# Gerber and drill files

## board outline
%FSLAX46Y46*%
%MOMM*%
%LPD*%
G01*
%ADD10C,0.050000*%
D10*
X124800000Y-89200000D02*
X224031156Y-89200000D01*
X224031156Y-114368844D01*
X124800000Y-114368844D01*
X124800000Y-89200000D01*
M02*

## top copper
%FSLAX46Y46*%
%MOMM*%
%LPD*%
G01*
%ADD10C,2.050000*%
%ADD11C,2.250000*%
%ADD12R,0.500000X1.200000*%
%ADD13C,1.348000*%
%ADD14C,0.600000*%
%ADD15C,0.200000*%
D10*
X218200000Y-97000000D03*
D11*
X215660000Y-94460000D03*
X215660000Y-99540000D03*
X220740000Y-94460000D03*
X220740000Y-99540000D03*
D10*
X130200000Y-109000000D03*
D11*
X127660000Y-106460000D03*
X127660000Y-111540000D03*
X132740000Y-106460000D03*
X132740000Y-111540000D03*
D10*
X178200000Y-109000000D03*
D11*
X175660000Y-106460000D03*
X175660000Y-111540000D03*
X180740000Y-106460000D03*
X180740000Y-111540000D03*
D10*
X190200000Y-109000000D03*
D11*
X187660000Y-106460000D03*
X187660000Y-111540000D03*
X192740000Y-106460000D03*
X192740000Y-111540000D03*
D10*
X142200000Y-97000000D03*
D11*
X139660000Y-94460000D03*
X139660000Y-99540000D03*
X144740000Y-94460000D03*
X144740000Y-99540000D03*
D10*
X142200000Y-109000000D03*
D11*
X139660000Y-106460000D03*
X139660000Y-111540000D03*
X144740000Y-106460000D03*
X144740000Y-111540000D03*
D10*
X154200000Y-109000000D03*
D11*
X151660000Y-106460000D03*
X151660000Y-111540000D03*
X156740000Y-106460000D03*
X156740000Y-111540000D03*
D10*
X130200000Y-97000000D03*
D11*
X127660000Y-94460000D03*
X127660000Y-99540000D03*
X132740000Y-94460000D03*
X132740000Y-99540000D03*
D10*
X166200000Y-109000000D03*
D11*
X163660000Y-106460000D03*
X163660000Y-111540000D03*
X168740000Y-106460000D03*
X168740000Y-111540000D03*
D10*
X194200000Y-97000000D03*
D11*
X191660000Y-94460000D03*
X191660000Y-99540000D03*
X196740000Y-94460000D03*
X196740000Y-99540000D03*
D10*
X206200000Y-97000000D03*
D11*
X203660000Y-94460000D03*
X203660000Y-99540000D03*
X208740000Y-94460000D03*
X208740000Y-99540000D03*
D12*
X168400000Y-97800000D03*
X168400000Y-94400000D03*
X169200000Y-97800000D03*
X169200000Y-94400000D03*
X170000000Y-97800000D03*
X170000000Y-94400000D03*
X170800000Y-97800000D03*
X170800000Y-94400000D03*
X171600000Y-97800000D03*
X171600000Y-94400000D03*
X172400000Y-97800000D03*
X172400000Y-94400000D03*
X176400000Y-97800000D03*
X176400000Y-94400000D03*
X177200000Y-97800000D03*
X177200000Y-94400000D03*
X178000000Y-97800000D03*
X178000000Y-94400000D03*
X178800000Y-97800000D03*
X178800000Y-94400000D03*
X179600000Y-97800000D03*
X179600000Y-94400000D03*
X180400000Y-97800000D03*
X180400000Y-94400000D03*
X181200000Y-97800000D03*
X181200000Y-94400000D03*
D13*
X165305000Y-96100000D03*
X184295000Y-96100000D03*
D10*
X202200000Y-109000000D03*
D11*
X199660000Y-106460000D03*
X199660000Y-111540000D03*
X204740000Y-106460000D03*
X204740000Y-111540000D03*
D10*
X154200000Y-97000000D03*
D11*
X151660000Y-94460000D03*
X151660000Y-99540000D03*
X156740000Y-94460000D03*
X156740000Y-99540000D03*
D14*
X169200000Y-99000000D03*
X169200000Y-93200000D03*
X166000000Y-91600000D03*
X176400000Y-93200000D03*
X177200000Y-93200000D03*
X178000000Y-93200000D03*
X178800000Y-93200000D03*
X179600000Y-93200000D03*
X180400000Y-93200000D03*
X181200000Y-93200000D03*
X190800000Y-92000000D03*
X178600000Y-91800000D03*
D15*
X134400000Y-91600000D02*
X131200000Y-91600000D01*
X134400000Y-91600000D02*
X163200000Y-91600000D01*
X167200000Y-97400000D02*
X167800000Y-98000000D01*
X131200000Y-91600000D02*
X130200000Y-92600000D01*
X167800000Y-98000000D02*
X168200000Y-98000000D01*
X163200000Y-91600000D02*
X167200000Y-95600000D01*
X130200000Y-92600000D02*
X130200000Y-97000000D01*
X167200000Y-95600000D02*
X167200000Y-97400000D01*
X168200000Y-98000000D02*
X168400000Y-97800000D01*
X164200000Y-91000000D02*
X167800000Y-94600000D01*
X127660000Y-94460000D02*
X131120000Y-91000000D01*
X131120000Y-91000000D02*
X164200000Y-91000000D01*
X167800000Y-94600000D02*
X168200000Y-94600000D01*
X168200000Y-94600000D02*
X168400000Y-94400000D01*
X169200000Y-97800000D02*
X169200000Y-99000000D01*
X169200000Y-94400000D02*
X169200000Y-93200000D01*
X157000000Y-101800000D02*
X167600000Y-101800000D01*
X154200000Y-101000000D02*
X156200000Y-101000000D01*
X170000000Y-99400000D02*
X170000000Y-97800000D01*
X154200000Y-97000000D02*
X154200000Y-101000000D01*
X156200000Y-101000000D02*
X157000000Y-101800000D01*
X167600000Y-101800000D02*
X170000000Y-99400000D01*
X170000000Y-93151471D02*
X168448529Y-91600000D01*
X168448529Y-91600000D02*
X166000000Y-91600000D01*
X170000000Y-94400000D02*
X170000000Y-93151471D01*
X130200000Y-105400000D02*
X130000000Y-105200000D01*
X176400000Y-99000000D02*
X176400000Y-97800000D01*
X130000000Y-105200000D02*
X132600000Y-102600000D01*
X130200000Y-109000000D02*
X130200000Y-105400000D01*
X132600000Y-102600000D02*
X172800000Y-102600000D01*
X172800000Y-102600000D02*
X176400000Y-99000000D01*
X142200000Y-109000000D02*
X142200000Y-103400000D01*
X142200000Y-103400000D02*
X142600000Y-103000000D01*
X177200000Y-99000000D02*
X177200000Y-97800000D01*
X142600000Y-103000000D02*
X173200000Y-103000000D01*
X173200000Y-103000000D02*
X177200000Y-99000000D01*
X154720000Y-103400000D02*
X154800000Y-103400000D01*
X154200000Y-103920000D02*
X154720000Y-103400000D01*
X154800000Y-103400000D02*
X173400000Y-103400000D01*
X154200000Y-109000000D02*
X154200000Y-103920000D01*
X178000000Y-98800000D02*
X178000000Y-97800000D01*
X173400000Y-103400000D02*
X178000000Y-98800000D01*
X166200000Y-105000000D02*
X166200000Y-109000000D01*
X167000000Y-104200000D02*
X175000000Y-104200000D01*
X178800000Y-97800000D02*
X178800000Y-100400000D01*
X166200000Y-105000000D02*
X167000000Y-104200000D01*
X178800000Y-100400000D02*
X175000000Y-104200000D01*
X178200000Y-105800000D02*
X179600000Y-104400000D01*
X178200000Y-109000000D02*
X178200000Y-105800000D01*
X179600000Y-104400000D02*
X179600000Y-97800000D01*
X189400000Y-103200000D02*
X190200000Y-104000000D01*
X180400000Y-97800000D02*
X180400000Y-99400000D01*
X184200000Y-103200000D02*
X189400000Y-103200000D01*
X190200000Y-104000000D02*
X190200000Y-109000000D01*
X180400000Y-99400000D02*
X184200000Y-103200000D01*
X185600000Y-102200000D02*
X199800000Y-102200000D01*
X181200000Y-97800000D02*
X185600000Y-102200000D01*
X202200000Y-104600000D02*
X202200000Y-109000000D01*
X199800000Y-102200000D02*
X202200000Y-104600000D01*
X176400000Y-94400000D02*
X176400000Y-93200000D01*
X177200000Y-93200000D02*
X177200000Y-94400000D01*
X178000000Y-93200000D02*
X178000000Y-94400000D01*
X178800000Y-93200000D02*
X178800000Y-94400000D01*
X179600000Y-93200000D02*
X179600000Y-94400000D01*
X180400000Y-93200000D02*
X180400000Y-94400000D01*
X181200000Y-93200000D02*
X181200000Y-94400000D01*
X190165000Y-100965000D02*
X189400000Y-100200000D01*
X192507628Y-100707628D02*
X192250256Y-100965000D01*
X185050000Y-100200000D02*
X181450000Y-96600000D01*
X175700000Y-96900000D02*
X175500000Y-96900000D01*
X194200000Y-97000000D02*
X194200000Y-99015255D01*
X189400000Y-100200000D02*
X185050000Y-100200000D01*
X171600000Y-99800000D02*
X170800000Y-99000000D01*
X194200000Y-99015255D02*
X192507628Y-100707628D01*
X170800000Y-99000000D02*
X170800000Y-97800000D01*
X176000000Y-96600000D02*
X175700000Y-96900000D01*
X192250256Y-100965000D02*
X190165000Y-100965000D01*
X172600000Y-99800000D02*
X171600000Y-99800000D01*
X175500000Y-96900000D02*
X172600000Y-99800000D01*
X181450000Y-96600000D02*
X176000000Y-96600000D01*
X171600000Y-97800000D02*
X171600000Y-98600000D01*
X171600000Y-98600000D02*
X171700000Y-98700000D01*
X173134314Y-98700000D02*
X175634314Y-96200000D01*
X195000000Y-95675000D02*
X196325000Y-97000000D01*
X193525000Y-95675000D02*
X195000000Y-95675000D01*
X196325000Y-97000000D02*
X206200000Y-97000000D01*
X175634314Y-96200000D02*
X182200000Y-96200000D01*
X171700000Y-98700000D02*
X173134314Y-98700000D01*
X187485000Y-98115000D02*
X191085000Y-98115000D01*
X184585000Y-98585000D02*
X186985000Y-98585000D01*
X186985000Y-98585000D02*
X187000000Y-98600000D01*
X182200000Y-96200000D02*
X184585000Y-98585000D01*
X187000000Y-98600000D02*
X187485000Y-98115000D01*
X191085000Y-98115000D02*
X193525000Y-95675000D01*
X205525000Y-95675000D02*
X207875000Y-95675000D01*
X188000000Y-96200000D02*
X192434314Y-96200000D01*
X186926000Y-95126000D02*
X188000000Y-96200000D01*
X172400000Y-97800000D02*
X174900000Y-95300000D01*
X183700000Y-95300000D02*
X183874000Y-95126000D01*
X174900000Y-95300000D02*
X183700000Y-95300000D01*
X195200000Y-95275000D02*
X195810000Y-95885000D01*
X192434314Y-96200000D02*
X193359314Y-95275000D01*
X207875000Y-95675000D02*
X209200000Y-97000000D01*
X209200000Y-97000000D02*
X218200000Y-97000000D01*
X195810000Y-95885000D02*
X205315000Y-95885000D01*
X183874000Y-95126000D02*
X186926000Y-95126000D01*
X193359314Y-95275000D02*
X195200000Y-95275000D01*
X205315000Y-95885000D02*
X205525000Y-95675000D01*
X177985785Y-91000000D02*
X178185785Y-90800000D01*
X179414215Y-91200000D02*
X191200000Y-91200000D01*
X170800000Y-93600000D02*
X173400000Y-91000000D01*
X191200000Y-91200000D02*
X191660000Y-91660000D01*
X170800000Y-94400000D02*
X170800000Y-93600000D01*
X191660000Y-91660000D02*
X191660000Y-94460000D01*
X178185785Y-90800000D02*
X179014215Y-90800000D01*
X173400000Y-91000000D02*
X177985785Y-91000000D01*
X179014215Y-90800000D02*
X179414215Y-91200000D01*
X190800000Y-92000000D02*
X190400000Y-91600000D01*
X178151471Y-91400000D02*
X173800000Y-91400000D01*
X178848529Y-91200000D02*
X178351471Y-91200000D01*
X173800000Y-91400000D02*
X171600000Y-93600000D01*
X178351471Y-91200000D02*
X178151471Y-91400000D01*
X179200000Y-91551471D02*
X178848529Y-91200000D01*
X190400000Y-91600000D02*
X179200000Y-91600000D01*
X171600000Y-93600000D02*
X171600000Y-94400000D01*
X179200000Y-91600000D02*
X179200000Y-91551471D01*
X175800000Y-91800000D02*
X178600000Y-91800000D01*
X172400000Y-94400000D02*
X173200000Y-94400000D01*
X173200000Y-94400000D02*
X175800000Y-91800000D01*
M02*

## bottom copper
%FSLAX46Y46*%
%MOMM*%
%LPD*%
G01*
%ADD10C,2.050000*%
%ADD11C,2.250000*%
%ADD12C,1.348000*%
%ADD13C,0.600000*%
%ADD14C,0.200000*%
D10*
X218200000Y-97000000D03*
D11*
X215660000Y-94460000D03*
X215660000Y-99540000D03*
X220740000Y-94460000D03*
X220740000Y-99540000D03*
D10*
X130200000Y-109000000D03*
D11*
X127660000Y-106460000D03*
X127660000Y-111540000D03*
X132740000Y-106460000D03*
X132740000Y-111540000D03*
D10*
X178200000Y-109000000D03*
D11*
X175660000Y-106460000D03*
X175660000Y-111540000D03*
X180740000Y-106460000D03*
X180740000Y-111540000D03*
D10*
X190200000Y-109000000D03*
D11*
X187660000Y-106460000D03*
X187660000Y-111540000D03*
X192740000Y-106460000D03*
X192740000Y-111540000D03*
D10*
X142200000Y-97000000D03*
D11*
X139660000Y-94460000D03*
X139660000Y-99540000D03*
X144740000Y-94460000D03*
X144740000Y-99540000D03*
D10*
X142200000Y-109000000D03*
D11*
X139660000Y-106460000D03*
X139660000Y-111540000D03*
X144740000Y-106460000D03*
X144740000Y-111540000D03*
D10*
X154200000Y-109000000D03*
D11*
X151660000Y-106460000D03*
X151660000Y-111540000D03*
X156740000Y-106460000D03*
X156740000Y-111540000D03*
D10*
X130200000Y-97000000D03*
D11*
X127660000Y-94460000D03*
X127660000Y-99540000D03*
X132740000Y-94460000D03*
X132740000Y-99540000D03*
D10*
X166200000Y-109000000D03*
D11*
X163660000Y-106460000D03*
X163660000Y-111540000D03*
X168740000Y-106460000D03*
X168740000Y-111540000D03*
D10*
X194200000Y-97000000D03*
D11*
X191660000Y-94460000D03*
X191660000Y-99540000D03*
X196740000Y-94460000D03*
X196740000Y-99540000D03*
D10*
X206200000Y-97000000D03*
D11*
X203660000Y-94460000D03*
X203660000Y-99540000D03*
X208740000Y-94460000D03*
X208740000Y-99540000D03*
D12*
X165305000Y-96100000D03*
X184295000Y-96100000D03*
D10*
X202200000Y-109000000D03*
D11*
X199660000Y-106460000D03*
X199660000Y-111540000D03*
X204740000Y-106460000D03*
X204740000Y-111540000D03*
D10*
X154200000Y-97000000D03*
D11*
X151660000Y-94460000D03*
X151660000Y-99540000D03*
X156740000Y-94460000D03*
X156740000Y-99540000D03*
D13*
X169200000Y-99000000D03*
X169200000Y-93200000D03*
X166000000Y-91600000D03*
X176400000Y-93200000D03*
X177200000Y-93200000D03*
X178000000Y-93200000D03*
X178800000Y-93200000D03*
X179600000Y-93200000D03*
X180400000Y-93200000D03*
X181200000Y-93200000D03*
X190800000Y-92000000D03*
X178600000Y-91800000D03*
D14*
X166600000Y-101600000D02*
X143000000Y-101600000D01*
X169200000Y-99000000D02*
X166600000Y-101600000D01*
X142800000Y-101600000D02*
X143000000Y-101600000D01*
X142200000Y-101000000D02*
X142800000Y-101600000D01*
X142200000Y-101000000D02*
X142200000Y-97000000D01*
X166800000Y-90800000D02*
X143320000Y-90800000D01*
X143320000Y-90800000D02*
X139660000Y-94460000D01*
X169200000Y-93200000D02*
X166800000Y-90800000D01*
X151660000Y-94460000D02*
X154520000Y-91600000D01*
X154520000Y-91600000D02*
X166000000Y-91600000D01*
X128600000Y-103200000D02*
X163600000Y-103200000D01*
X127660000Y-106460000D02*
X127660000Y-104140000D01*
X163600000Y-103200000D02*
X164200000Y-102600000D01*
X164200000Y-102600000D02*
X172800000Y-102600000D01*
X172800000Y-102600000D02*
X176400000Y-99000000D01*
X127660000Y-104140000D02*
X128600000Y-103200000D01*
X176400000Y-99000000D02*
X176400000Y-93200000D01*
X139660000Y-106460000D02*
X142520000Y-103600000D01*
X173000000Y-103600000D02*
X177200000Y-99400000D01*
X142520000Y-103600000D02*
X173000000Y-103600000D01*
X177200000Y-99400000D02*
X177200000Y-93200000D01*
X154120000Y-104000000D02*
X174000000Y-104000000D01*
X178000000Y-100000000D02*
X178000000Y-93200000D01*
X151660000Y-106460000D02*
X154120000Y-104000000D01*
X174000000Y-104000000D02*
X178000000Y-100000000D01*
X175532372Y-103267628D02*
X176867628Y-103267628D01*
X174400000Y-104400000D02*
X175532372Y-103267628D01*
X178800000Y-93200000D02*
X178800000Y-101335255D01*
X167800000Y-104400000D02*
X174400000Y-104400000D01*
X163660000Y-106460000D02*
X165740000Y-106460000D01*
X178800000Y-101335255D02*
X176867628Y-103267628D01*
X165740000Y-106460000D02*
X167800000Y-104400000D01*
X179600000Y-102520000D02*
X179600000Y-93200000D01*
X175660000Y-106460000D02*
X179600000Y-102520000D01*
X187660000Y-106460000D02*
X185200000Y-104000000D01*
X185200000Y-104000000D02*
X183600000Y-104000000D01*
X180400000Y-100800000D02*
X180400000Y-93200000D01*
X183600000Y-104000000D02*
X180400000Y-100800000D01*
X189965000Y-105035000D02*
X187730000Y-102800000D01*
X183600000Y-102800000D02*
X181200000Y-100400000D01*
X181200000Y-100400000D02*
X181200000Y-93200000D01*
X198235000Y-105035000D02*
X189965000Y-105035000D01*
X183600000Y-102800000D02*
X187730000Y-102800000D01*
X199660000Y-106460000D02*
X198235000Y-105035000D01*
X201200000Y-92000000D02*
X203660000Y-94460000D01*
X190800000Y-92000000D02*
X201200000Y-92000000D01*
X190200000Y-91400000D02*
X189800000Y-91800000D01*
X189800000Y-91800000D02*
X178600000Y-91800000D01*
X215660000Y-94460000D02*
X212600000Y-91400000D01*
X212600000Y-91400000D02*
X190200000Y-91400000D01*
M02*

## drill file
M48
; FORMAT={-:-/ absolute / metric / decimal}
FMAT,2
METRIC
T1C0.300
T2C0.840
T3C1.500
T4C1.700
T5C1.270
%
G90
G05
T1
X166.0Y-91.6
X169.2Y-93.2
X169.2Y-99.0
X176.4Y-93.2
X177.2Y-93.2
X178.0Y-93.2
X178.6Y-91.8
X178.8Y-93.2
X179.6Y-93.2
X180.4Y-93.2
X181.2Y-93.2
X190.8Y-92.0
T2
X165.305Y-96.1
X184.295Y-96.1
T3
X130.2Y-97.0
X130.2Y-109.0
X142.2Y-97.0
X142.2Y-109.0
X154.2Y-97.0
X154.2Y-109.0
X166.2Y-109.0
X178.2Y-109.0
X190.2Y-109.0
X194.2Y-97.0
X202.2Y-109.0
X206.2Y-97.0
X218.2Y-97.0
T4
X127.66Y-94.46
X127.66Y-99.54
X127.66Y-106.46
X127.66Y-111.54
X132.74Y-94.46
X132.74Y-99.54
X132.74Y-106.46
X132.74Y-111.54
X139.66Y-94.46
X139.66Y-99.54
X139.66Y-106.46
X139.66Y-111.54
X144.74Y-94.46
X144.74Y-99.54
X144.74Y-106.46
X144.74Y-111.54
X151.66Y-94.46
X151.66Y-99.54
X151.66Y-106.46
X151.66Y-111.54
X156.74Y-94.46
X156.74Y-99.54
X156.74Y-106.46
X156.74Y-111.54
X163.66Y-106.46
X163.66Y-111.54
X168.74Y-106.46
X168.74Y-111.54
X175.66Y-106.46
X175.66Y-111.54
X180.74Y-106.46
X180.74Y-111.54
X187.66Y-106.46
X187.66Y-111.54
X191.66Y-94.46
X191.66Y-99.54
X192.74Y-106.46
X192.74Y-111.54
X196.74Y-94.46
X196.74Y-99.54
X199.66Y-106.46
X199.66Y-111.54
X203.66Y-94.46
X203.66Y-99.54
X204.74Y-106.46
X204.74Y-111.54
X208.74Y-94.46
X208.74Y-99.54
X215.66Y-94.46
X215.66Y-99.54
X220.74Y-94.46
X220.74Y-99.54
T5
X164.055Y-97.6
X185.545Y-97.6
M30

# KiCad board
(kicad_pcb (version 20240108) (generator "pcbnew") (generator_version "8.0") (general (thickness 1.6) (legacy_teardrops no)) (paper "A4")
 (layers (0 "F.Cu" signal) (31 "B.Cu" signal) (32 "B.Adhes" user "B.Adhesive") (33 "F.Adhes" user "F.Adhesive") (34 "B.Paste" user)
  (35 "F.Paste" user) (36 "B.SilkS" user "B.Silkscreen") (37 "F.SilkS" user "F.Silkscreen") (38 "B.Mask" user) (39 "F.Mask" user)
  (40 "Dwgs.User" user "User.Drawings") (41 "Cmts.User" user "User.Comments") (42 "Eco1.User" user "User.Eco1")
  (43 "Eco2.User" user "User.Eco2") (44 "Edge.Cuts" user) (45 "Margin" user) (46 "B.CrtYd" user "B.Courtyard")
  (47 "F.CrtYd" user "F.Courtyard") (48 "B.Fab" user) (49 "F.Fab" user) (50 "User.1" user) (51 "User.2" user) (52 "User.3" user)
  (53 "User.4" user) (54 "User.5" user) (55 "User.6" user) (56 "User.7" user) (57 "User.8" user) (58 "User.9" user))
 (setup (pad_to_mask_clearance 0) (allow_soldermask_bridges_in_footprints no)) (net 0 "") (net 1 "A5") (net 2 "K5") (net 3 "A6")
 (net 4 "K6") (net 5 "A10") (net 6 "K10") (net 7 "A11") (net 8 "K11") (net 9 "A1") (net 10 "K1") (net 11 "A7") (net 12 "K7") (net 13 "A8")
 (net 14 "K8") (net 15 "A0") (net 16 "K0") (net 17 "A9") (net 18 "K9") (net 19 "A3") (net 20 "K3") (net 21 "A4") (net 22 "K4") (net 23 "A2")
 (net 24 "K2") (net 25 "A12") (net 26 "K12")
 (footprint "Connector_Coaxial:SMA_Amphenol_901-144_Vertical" (layer "F.Cu") (at 218.2 97)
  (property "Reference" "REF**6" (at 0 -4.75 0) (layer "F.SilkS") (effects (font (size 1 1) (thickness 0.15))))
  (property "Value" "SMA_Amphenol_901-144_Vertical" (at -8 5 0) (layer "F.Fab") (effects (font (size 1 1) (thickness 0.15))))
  (pad "1" thru_hole circle (at 0 0) (size 2.05 2.05) (drill 1.5) (layers "*.Cu" "*.Mask") (remove_unused_layers no) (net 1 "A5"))
  (pad "2" thru_hole circle (at -2.54 -2.54) (size 2.25 2.25) (drill 1.7) (layers "*.Cu" "*.Mask") (remove_unused_layers no) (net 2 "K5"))
  (pad "2" thru_hole circle (at -2.54 2.54) (size 2.25 2.25) (drill 1.7) (layers "*.Cu" "*.Mask") (remove_unused_layers no))
  (pad "2" thru_hole circle (at 2.54 -2.54) (size 2.25 2.25) (drill 1.7) (layers "*.Cu" "*.Mask") (remove_unused_layers no))
  (pad "2" thru_hole circle (at 2.54 2.54) (size 2.25 2.25) (drill 1.7) (layers "*.Cu" "*.Mask") (remove_unused_layers no)))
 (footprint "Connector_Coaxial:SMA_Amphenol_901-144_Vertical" (layer "F.Cu") (at 130.2 109)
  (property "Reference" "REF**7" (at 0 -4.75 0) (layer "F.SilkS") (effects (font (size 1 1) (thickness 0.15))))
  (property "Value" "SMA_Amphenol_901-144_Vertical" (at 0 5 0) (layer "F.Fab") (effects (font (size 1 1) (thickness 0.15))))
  (pad "1" thru_hole circle (at 0 0) (size 2.05 2.05) (drill 1.5) (layers "*.Cu" "*.Mask") (remove_unused_layers no) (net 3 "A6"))
  (pad "2" thru_hole circle (at -2.54 -2.54) (size 2.25 2.25) (drill 1.7) (layers "*.Cu" "*.Mask") (remove_unused_layers no) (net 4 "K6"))
  (pad "2" thru_hole circle (at -2.54 2.54) (size 2.25 2.25) (drill 1.7) (layers "*.Cu" "*.Mask") (remove_unused_layers no))
  (pad "2" thru_hole circle (at 2.54 -2.54) (size 2.25 2.25) (drill 1.7) (layers "*.Cu" "*.Mask") (remove_unused_layers no))
  (pad "2" thru_hole circle (at 2.54 2.54) (size 2.25 2.25) (drill 1.7) (layers "*.Cu" "*.Mask") (remove_unused_layers no)))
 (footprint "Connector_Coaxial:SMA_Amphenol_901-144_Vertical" (layer "F.Cu") (at 178.2 109)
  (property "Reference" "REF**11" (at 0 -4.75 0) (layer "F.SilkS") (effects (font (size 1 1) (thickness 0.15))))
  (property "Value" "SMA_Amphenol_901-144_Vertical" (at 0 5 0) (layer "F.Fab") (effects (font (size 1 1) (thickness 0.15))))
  (pad "1" thru_hole circle (at 0 0) (size 2.05 2.05) (drill 1.5) (layers "*.Cu" "*.Mask") (remove_unused_layers no) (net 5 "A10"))
  (pad "2" thru_hole circle (at -2.54 -2.54) (size 2.25 2.25) (drill 1.7) (layers "*.Cu" "*.Mask") (remove_unused_layers no) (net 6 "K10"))
  (pad "2" thru_hole circle (at -2.54 2.54) (size 2.25 2.25) (drill 1.7) (layers "*.Cu" "*.Mask") (remove_unused_layers no))
  (pad "2" thru_hole circle (at 2.54 -2.54) (size 2.25 2.25) (drill 1.7) (layers "*.Cu" "*.Mask") (remove_unused_layers no))
  (pad "2" thru_hole circle (at 2.54 2.54) (size 2.25 2.25) (drill 1.7) (layers "*.Cu" "*.Mask") (remove_unused_layers no)))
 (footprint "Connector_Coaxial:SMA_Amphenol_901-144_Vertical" (layer "F.Cu") (at 190.2 109)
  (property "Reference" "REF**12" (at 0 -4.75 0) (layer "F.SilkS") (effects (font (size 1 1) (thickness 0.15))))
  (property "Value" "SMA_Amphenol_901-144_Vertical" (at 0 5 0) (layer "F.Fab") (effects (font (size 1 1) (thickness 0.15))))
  (pad "1" thru_hole circle (at 0 0) (size 2.05 2.05) (drill 1.5) (layers "*.Cu" "*.Mask") (remove_unused_layers no) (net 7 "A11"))
  (pad "2" thru_hole circle (at -2.54 -2.54) (size 2.25 2.25) (drill 1.7) (layers "*.Cu" "*.Mask") (remove_unused_layers no) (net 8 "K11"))
  (pad "2" thru_hole circle (at -2.54 2.54) (size 2.25 2.25) (drill 1.7) (layers "*.Cu" "*.Mask") (remove_unused_layers no))
  (pad "2" thru_hole circle (at 2.54 -2.54) (size 2.25 2.25) (drill 1.7) (layers "*.Cu" "*.Mask") (remove_unused_layers no))
  (pad "2" thru_hole circle (at 2.54 2.54) (size 2.25 2.25) (drill 1.7) (layers "*.Cu" "*.Mask") (remove_unused_layers no)))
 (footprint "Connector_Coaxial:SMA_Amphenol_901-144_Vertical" (layer "F.Cu") (at 142.2 97)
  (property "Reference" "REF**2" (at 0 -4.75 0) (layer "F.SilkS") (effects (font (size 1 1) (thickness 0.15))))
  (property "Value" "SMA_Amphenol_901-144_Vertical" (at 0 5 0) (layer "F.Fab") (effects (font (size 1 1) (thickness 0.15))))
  (pad "1" thru_hole circle (at 0 0) (size 2.05 2.05) (drill 1.5) (layers "*.Cu" "*.Mask") (remove_unused_layers no) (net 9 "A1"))
  (pad "2" thru_hole circle (at -2.54 -2.54) (size 2.25 2.25) (drill 1.7) (layers "*.Cu" "*.Mask") (remove_unused_layers no) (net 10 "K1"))
  (pad "2" thru_hole circle (at -2.54 2.54) (size 2.25 2.25) (drill 1.7) (layers "*.Cu" "*.Mask") (remove_unused_layers no))
  (pad "2" thru_hole circle (at 2.54 -2.54) (size 2.25 2.25) (drill 1.7) (layers "*.Cu" "*.Mask") (remove_unused_layers no))
  (pad "2" thru_hole circle (at 2.54 2.54) (size 2.25 2.25) (drill 1.7) (layers "*.Cu" "*.Mask") (remove_unused_layers no)))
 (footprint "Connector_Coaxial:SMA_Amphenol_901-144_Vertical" (layer "F.Cu") (at 142.2 109)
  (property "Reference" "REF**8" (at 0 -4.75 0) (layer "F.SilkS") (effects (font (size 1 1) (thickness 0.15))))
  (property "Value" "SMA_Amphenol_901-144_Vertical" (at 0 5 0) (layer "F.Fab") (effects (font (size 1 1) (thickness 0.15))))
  (pad "1" thru_hole circle (at 0 0) (size 2.05 2.05) (drill 1.5) (layers "*.Cu" "*.Mask") (remove_unused_layers no) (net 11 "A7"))
  (pad "2" thru_hole circle (at -2.54 -2.54) (size 2.25 2.25) (drill 1.7) (layers "*.Cu" "*.Mask") (remove_unused_layers no) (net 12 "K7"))
  (pad "2" thru_hole circle (at -2.54 2.54) (size 2.25 2.25) (drill 1.7) (layers "*.Cu" "*.Mask") (remove_unused_layers no))
  (pad "2" thru_hole circle (at 2.54 -2.54) (size 2.25 2.25) (drill 1.7) (layers "*.Cu" "*.Mask") (remove_unused_layers no))
  (pad "2" thru_hole circle (at 2.54 2.54) (size 2.25 2.25) (drill 1.7) (layers "*.Cu" "*.Mask") (remove_unused_layers no)))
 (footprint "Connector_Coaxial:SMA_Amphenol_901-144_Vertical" (layer "F.Cu") (at 154.2 109)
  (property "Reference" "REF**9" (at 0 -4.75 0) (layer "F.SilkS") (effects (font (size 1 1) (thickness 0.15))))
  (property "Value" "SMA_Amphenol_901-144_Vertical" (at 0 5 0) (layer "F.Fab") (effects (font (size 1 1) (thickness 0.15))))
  (pad "1" thru_hole circle (at 0 0) (size 2.05 2.05) (drill 1.5) (layers "*.Cu" "*.Mask") (remove_unused_layers no) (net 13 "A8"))
  (pad "2" thru_hole circle (at -2.54 -2.54) (size 2.25 2.25) (drill 1.7) (layers "*.Cu" "*.Mask") (remove_unused_layers no) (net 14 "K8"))
  (pad "2" thru_hole circle (at -2.54 2.54) (size 2.25 2.25) (drill 1.7) (layers "*.Cu" "*.Mask") (remove_unused_layers no))
  (pad "2" thru_hole circle (at 2.54 -2.54) (size 2.25 2.25) (drill 1.7) (layers "*.Cu" "*.Mask") (remove_unused_layers no))
  (pad "2" thru_hole circle (at 2.54 2.54) (size 2.25 2.25) (drill 1.7) (layers "*.Cu" "*.Mask") (remove_unused_layers no)))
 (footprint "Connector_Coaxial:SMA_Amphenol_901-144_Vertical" (layer "F.Cu") (at 130.2 97)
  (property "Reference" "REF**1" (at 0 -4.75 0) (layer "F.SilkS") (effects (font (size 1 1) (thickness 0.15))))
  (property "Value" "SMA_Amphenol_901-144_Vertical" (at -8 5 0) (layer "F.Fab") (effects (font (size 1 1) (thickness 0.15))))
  (pad "1" thru_hole circle (at 0 0) (size 2.05 2.05) (drill 1.5) (layers "*.Cu" "*.Mask") (remove_unused_layers no) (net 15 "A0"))
  (pad "2" thru_hole circle (at -2.54 -2.54) (size 2.25 2.25) (drill 1.7) (layers "*.Cu" "*.Mask") (remove_unused_layers no) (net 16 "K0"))
  (pad "2" thru_hole circle (at -2.54 2.54) (size 2.25 2.25) (drill 1.7) (layers "*.Cu" "*.Mask") (remove_unused_layers no))
  (pad "2" thru_hole circle (at 2.54 -2.54) (size 2.25 2.25) (drill 1.7) (layers "*.Cu" "*.Mask") (remove_unused_layers no))
  (pad "2" thru_hole circle (at 2.54 2.54) (size 2.25 2.25) (drill 1.7) (layers "*.Cu" "*.Mask") (remove_unused_layers no)))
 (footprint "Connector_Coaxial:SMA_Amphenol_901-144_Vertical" (layer "F.Cu") (at 166.2 109)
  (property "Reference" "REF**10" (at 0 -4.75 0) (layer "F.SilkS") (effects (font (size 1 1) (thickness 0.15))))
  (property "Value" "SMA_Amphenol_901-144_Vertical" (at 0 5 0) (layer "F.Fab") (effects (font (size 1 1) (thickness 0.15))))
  (pad "1" thru_hole circle (at 0 0) (size 2.05 2.05) (drill 1.5) (layers "*.Cu" "*.Mask") (remove_unused_layers no) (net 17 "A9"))
  (pad "2" thru_hole circle (at -2.54 -2.54) (size 2.25 2.25) (drill 1.7) (layers "*.Cu" "*.Mask") (remove_unused_layers no) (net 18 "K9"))
  (pad "2" thru_hole circle (at -2.54 2.54) (size 2.25 2.25) (drill 1.7) (layers "*.Cu" "*.Mask") (remove_unused_layers no))
  (pad "2" thru_hole circle (at 2.54 -2.54) (size 2.25 2.25) (drill 1.7) (layers "*.Cu" "*.Mask") (remove_unused_layers no))
  (pad "2" thru_hole circle (at 2.54 2.54) (size 2.25 2.25) (drill 1.7) (layers "*.Cu" "*.Mask") (remove_unused_layers no)))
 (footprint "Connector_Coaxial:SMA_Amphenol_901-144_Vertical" (layer "F.Cu") (at 194.2 97)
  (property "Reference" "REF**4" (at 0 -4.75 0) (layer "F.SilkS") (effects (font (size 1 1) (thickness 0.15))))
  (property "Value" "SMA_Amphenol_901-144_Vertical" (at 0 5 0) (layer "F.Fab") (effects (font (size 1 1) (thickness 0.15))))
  (pad "1" thru_hole circle (at 0 0) (size 2.05 2.05) (drill 1.5) (layers "*.Cu" "*.Mask") (remove_unused_layers no) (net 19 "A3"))
  (pad "2" thru_hole circle (at -2.54 -2.54) (size 2.25 2.25) (drill 1.7) (layers "*.Cu" "*.Mask") (remove_unused_layers no) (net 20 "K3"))
  (pad "2" thru_hole circle (at -2.54 2.54) (size 2.25 2.25) (drill 1.7) (layers "*.Cu" "*.Mask") (remove_unused_layers no))
  (pad "2" thru_hole circle (at 2.54 -2.54) (size 2.25 2.25) (drill 1.7) (layers "*.Cu" "*.Mask") (remove_unused_layers no))
  (pad "2" thru_hole circle (at 2.54 2.54) (size 2.25 2.25) (drill 1.7) (layers "*.Cu" "*.Mask") (remove_unused_layers no)))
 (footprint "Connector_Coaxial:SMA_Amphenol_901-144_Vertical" (layer "F.Cu") (at 206.2 97)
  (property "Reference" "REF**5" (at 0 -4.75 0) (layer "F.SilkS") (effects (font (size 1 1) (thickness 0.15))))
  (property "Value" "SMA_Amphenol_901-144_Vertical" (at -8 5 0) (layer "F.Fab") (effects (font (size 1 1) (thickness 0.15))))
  (pad "1" thru_hole circle (at 0 0) (size 2.05 2.05) (drill 1.5) (layers "*.Cu" "*.Mask") (remove_unused_layers no) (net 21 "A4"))
  (pad "2" thru_hole circle (at -2.54 -2.54) (size 2.25 2.25) (drill 1.7) (layers "*.Cu" "*.Mask") (remove_unused_layers no) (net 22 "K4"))
  (pad "2" thru_hole circle (at -2.54 2.54) (size 2.25 2.25) (drill 1.7) (layers "*.Cu" "*.Mask") (remove_unused_layers no))
  (pad "2" thru_hole circle (at 2.54 -2.54) (size 2.25 2.25) (drill 1.7) (layers "*.Cu" "*.Mask") (remove_unused_layers no))
  (pad "2" thru_hole circle (at 2.54 2.54) (size 2.25 2.25) (drill 1.7) (layers "*.Cu" "*.Mask") (remove_unused_layers no)))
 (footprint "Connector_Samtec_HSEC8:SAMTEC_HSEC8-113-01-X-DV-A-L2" (layer "F.Cu") (at 174.8 96.1)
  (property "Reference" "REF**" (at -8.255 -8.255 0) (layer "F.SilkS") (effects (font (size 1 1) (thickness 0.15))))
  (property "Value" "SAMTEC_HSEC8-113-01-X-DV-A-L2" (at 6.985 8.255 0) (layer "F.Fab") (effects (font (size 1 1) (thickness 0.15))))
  (pad "" np_thru_hole circle (at -10.745 1.5) (size 1.27 1.27) (drill 1.27) (layers "F&B.Cu" "*.Mask"))
  (pad "" np_thru_hole circle (at 10.745 1.5) (size 1.27 1.27) (drill 1.27) (layers "F&B.Cu" "*.Mask"))
  (pad "01" smd rect (at -6.4 1.7) (size 0.5 1.2) (layers "F.Cu" "F.Paste" "F.Mask") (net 15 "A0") (solder_mask_margin 0.102))
  (pad "02" smd rect (at -6.4 -1.7) (size 0.5 1.2) (layers "F.Cu" "F.Paste" "F.Mask") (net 16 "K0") (solder_mask_margin 0.102))
  (pad "02" smd rect (at -5.6 1.7) (size 0.5 1.2) (layers "F.Cu" "F.Paste" "F.Mask") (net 9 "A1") (solder_mask_margin 0.102))
  (pad "04" smd rect (at -5.6 -1.7) (size 0.5 1.2) (layers "F.Cu" "F.Paste" "F.Mask") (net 10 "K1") (solder_mask_margin 0.102))
  (pad "05" smd rect (at -4.8 1.7) (size 0.5 1.2) (layers "F.Cu" "F.Paste" "F.Mask") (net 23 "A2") (solder_mask_margin 0.102))
  (pad "06" smd rect (at -4.8 -1.7) (size 0.5 1.2) (layers "F.Cu" "F.Paste" "F.Mask") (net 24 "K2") (solder_mask_margin 0.102))
  (pad "07" smd rect (at -4 1.7) (size 0.5 1.2) (layers "F.Cu" "F.Paste" "F.Mask") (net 19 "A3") (solder_mask_margin 0.102))
  (pad "08" smd rect (at -4 -1.7) (size 0.5 1.2) (layers "F.Cu" "F.Paste" "F.Mask") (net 20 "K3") (solder_mask_margin 0.102))
  (pad "09" smd rect (at -3.2 1.7) (size 0.5 1.2) (layers "F.Cu" "F.Paste" "F.Mask") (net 21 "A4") (solder_mask_margin 0.102))
  (pad "10" smd rect (at -3.2 -1.7) (size 0.5 1.2) (layers "F.Cu" "F.Paste" "F.Mask") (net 22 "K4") (solder_mask_margin 0.102))
  (pad "11" smd rect (at -2.4 1.7) (size 0.5 1.2) (layers "F.Cu" "F.Paste" "F.Mask") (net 1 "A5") (solder_mask_margin 0.102))
  (pad "12" smd rect (at -2.4 -1.7) (size 0.5 1.2) (layers "F.Cu" "F.Paste" "F.Mask") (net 2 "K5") (solder_mask_margin 0.102))
  (pad "13" smd rect (at 1.6 1.7) (size 0.5 1.2) (layers "F.Cu" "F.Paste" "F.Mask") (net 3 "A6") (solder_mask_margin 0.102))
  (pad "14" smd rect (at 1.6 -1.7) (size 0.5 1.2) (layers "F.Cu" "F.Paste" "F.Mask") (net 4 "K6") (solder_mask_margin 0.102))
  (pad "15" smd rect (at 2.4 1.7) (size 0.5 1.2) (layers "F.Cu" "F.Paste" "F.Mask") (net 11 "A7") (solder_mask_margin 0.102))
  (pad "16" smd rect (at 2.4 -1.7) (size 0.5 1.2) (layers "F.Cu" "F.Paste" "F.Mask") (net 12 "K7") (solder_mask_margin 0.102))
  (pad "17" smd rect (at 3.2 1.7) (size 0.5 1.2) (layers "F.Cu" "F.Paste" "F.Mask") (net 13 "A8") (solder_mask_margin 0.102))
  (pad "18" smd rect (at 3.2 -1.7) (size 0.5 1.2) (layers "F.Cu" "F.Paste" "F.Mask") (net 14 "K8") (solder_mask_margin 0.102))
  (pad "19" smd rect (at 4 1.7) (size 0.5 1.2) (layers "F.Cu" "F.Paste" "F.Mask") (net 17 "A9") (solder_mask_margin 0.102))
  (pad "20" smd rect (at 4 -1.7) (size 0.5 1.2) (layers "F.Cu" "F.Paste" "F.Mask") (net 18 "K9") (solder_mask_margin 0.102))
  (pad "21" smd rect (at 4.8 1.7) (size 0.5 1.2) (layers "F.Cu" "F.Paste" "F.Mask") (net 5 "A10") (solder_mask_margin 0.102))
  (pad "22" smd rect (at 4.8 -1.7) (size 0.5 1.2) (layers "F.Cu" "F.Paste" "F.Mask") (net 6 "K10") (solder_mask_margin 0.102))
  (pad "23" smd rect (at 5.6 1.7) (size 0.5 1.2) (layers "F.Cu" "F.Paste" "F.Mask") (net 7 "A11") (solder_mask_margin 0.102))
  (pad "24" smd rect (at 5.6 -1.7) (size 0.5 1.2) (layers "F.Cu" "F.Paste" "F.Mask") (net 8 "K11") (solder_mask_margin 0.102))
  (pad "25" smd rect (at 6.4 1.7) (size 0.5 1.2) (layers "F.Cu" "F.Paste" "F.Mask") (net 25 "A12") (solder_mask_margin 0.102))
  (pad "26" smd rect (at 6.4 -1.7) (size 0.5 1.2) (layers "F.Cu" "F.Paste" "F.Mask") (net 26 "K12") (solder_mask_margin 0.102))
  (pad "S1" thru_hole circle (at -9.495 0) (size 1.348 1.348) (drill 0.84) (layers "*.Cu" "*.Mask") (remove_unused_layers no)
   (solder_mask_margin 0.102))
  (pad "S2" thru_hole circle (at 9.495 0) (size 1.348 1.348) (drill 0.84) (layers "*.Cu" "*.Mask") (remove_unused_layers no)
   (solder_mask_margin 0.102)))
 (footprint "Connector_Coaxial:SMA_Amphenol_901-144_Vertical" (layer "F.Cu") (at 202.2 109)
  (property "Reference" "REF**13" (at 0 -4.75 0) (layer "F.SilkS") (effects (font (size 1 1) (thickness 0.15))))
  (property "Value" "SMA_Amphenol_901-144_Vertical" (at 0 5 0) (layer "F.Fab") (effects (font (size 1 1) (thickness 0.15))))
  (pad "1" thru_hole circle (at 0 0) (size 2.05 2.05) (drill 1.5) (layers "*.Cu" "*.Mask") (remove_unused_layers no) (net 25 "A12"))
  (pad "2" thru_hole circle (at -2.54 -2.54) (size 2.25 2.25) (drill 1.7) (layers "*.Cu" "*.Mask") (remove_unused_layers no) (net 26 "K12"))
  (pad "2" thru_hole circle (at -2.54 2.54) (size 2.25 2.25) (drill 1.7) (layers "*.Cu" "*.Mask") (remove_unused_layers no))
  (pad "2" thru_hole circle (at 2.54 -2.54) (size 2.25 2.25) (drill 1.7) (layers "*.Cu" "*.Mask") (remove_unused_layers no))
  (pad "2" thru_hole circle (at 2.54 2.54) (size 2.25 2.25) (drill 1.7) (layers "*.Cu" "*.Mask") (remove_unused_layers no)))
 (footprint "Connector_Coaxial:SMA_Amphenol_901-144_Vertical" (layer "F.Cu") (at 154.2 97)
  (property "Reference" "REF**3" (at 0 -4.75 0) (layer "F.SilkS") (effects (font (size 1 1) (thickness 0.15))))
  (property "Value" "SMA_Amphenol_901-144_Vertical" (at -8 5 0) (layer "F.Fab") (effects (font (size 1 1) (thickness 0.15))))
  (pad "1" thru_hole circle (at 0 0) (size 2.05 2.05) (drill 1.5) (layers "*.Cu" "*.Mask") (remove_unused_layers no) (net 23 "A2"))
  (pad "2" thru_hole circle (at -2.54 -2.54) (size 2.25 2.25) (drill 1.7) (layers "*.Cu" "*.Mask") (remove_unused_layers no) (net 24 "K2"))
  (pad "2" thru_hole circle (at -2.54 2.54) (size 2.25 2.25) (drill 1.7) (layers "*.Cu" "*.Mask") (remove_unused_layers no))
  (pad "2" thru_hole circle (at 2.54 -2.54) (size 2.25 2.25) (drill 1.7) (layers "*.Cu" "*.Mask") (remove_unused_layers no))
  (pad "2" thru_hole circle (at 2.54 2.54) (size 2.25 2.25) (drill 1.7) (layers "*.Cu" "*.Mask") (remove_unused_layers no)))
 (gr_rect (start 124.8 89.2) (end 224.031156 114.368844) (stroke (width 0.05) (type default)) (fill none) (layer "Edge.Cuts"))
 (segment (start 134.4 91.6) (end 131.2 91.6) (width 0.2) (layer "F.Cu") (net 15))
 (segment (start 134.4 91.6) (end 163.2 91.6) (width 0.2) (layer "F.Cu") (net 15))
 (segment (start 167.2 97.4) (end 167.8 98) (width 0.2) (layer "F.Cu") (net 15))
 (segment (start 131.2 91.6) (end 130.2 92.6) (width 0.2) (layer "F.Cu") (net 15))
 (segment (start 167.8 98) (end 168.2 98) (width 0.2) (layer "F.Cu") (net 15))
 (segment (start 163.2 91.6) (end 167.2 95.6) (width 0.2) (layer "F.Cu") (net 15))
 (segment (start 130.2 92.6) (end 130.2 97) (width 0.2) (layer "F.Cu") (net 15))
 (segment (start 167.2 95.6) (end 167.2 97.4) (width 0.2) (layer "F.Cu") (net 15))
 (segment (start 168.2 98) (end 168.4 97.8) (width 0.2) (layer "F.Cu") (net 15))
 (segment (start 164.2 91) (end 167.8 94.6) (width 0.2) (layer "F.Cu") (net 16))
 (segment (start 127.66 94.46) (end 131.12 91) (width 0.2) (layer "F.Cu") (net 16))
 (segment (start 131.12 91) (end 164.2 91) (width 0.2) (layer "F.Cu") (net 16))
 (segment (start 167.8 94.6) (end 168.2 94.6) (width 0.2) (layer "F.Cu") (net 16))
 (segment (start 168.2 94.6) (end 168.4 94.4) (width 0.2) (layer "F.Cu") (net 16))
 (segment (start 169.2 97.8) (end 169.2 99) (width 0.2) (layer "F.Cu") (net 9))
 (via (at 169.2 99) (size 0.6) (drill 0.3) (layers "F.Cu" "B.Cu") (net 9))
 (segment (start 166.6 101.6) (end 143 101.6) (width 0.2) (layer "B.Cu") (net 9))
 (segment (start 169.2 99) (end 166.6 101.6) (width 0.2) (layer "B.Cu") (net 9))
 (segment (start 142.8 101.6) (end 143 101.6) (width 0.2) (layer "B.Cu") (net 9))
 (segment (start 142.2 101) (end 142.8 101.6) (width 0.2) (layer "B.Cu") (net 9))
 (segment (start 142.2 101) (end 142.2 97) (width 0.2) (layer "B.Cu") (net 9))
 (segment (start 169.2 94.4) (end 169.2 93.2) (width 0.2) (layer "F.Cu") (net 10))
 (via (at 169.2 93.2) (size 0.6) (drill 0.3) (layers "F.Cu" "B.Cu") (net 10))
 (segment (start 166.8 90.8) (end 143.32 90.8) (width 0.2) (layer "B.Cu") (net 10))
 (segment (start 143.32 90.8) (end 139.66 94.46) (width 0.2) (layer "B.Cu") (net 10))
 (segment (start 169.2 93.2) (end 166.8 90.8) (width 0.2) (layer "B.Cu") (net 10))
 (segment (start 157 101.8) (end 167.6 101.8) (width 0.2) (layer "F.Cu") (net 23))
 (segment (start 154.2 101) (end 156.2 101) (width 0.2) (layer "F.Cu") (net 23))
 (segment (start 170 99.4) (end 170 97.8) (width 0.2) (layer "F.Cu") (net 23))
 (segment (start 154.2 97) (end 154.2 101) (width 0.2) (layer "F.Cu") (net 23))
 (segment (start 156.2 101) (end 157 101.8) (width 0.2) (layer "F.Cu") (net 23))
 (segment (start 167.6 101.8) (end 170 99.4) (width 0.2) (layer "F.Cu") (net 23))
 (segment (start 170 93.151471) (end 168.448529 91.6) (width 0.2) (layer "F.Cu") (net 24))
 (segment (start 168.448529 91.6) (end 166 91.6) (width 0.2) (layer "F.Cu") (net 24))
 (segment (start 170 94.4) (end 170 93.151471) (width 0.2) (layer "F.Cu") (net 24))
 (via (at 166 91.6) (size 0.6) (drill 0.3) (layers "F.Cu" "B.Cu") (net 24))
 (segment (start 151.66 94.46) (end 154.52 91.6) (width 0.2) (layer "B.Cu") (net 24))
 (segment (start 154.52 91.6) (end 166 91.6) (width 0.2) (layer "B.Cu") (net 24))
 (segment (start 130.2 105.4) (end 130 105.2) (width 0.2) (layer "F.Cu") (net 3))
 (segment (start 176.4 99) (end 176.4 97.8) (width 0.2) (layer "F.Cu") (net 3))
 (segment (start 130 105.2) (end 132.6 102.6) (width 0.2) (layer "F.Cu") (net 3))
 (segment (start 130.2 109) (end 130.2 105.4) (width 0.2) (layer "F.Cu") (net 3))
 (segment (start 132.6 102.6) (end 172.8 102.6) (width 0.2) (layer "F.Cu") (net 3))
 (segment (start 172.8 102.6) (end 176.4 99) (width 0.2) (layer "F.Cu") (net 3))
 (segment (start 142.2 109) (end 142.2 103.4) (width 0.2) (layer "F.Cu") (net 11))
 (segment (start 142.2 103.4) (end 142.6 103) (width 0.2) (layer "F.Cu") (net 11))
 (segment (start 177.2 99) (end 177.2 97.8) (width 0.2) (layer "F.Cu") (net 11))
 (segment (start 142.6 103) (end 173.2 103) (width 0.2) (layer "F.Cu") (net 11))
 (segment (start 173.2 103) (end 177.2 99) (width 0.2) (layer "F.Cu") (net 11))
 (segment (start 154.72 103.4) (end 154.8 103.4) (width 0.2) (layer "F.Cu") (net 13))
 (segment (start 154.2 103.92) (end 154.72 103.4) (width 0.2) (layer "F.Cu") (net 13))
 (segment (start 154.8 103.4) (end 173.4 103.4) (width 0.2) (layer "F.Cu") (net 13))
 (segment (start 154.2 109) (end 154.2 103.92) (width 0.2) (layer "F.Cu") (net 13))
 (segment (start 178 98.8) (end 178 97.8) (width 0.2) (layer "F.Cu") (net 13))
 (segment (start 173.4 103.4) (end 178 98.8) (width 0.2) (layer "F.Cu") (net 13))
 (segment (start 166.2 105) (end 166.2 109) (width 0.2) (layer "F.Cu") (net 17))
 (segment (start 167 104.2) (end 175 104.2) (width 0.2) (layer "F.Cu") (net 17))
 (segment (start 178.8 97.8) (end 178.8 100.4) (width 0.2) (layer "F.Cu") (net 17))
 (segment (start 166.2 105) (end 167 104.2) (width 0.2) (layer "F.Cu") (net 17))
 (segment (start 178.8 100.4) (end 175 104.2) (width 0.2) (layer "F.Cu") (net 17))
 (segment (start 178.2 105.8) (end 179.6 104.4) (width 0.2) (layer "F.Cu") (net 5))
 (segment (start 178.2 109) (end 178.2 105.8) (width 0.2) (layer "F.Cu") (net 5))
 (segment (start 179.6 104.4) (end 179.6 97.8) (width 0.2) (layer "F.Cu") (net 5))
 (segment (start 189.4 103.2) (end 190.2 104) (width 0.2) (layer "F.Cu") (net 7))
 (segment (start 180.4 97.8) (end 180.4 99.4) (width 0.2) (layer "F.Cu") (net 7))
 (segment (start 184.2 103.2) (end 189.4 103.2) (width 0.2) (layer "F.Cu") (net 7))
 (segment (start 190.2 104) (end 190.2 109) (width 0.2) (layer "F.Cu") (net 7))
 (segment (start 180.4 99.4) (end 184.2 103.2) (width 0.2) (layer "F.Cu") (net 7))
 (segment (start 185.6 102.2) (end 199.8 102.2) (width 0.2) (layer "F.Cu") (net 25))
 (segment (start 181.2 97.8) (end 185.6 102.2) (width 0.2) (layer "F.Cu") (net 25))
 (segment (start 202.2 104.6) (end 202.2 109) (width 0.2) (layer "F.Cu") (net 25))
 (segment (start 199.8 102.2) (end 202.2 104.6) (width 0.2) (layer "F.Cu") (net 25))
 (segment (start 176.4 94.4) (end 176.4 93.2) (width 0.2) (layer "F.Cu") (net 4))
 (via (at 176.4 93.2) (size 0.6) (drill 0.3) (layers "F.Cu" "B.Cu") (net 4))
 (segment (start 128.6 103.2) (end 163.6 103.2) (width 0.2) (layer "B.Cu") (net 4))
 (segment (start 127.66 106.46) (end 127.66 104.14) (width 0.2) (layer "B.Cu") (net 4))
 (segment (start 163.6 103.2) (end 164.2 102.6) (width 0.2) (layer "B.Cu") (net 4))
 (segment (start 164.2 102.6) (end 172.8 102.6) (width 0.2) (layer "B.Cu") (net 4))
 (segment (start 172.8 102.6) (end 176.4 99) (width 0.2) (layer "B.Cu") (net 4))
 (segment (start 127.66 104.14) (end 128.6 103.2) (width 0.2) (layer "B.Cu") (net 4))
 (segment (start 176.4 99) (end 176.4 93.2) (width 0.2) (layer "B.Cu") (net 4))
 (segment (start 177.2 93.2) (end 177.2 94.4) (width 0.2) (layer "F.Cu") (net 12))
 (via (at 177.2 93.2) (size 0.6) (drill 0.3) (layers "F.Cu" "B.Cu") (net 12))
 (segment (start 139.66 106.46) (end 142.52 103.6) (width 0.2) (layer "B.Cu") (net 12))
 (segment (start 173 103.6) (end 177.2 99.4) (width 0.2) (layer "B.Cu") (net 12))
 (segment (start 142.52 103.6) (end 173 103.6) (width 0.2) (layer "B.Cu") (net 12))
 (segment (start 177.2 99.4) (end 177.2 93.2) (width 0.2) (layer "B.Cu") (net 12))
 (segment (start 178 93.2) (end 178 94.4) (width 0.2) (layer "F.Cu") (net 14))
 (via (at 178 93.2) (size 0.6) (drill 0.3) (layers "F.Cu" "B.Cu") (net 14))
 (segment (start 154.12 104) (end 174 104) (width 0.2) (layer "B.Cu") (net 14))
 (segment (start 178 100) (end 178 93.2) (width 0.2) (layer "B.Cu") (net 14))
 (segment (start 151.66 106.46) (end 154.12 104) (width 0.2) (layer "B.Cu") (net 14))
 (segment (start 174 104) (end 178 100) (width 0.2) (layer "B.Cu") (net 14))
 (segment (start 178.8 93.2) (end 178.8 94.4) (width 0.2) (layer "F.Cu") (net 18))
 (via (at 178.8 93.2) (size 0.6) (drill 0.3) (layers "F.Cu" "B.Cu") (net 18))
 (segment (start 175.532372 103.267628) (end 176.867628 103.267628) (width 0.2) (layer "B.Cu") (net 18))
 (segment (start 174.4 104.4) (end 175.532372 103.267628) (width 0.2) (layer "B.Cu") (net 18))
 (segment (start 178.8 93.2) (end 178.8 101.335255) (width 0.2) (layer "B.Cu") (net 18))
 (segment (start 167.8 104.4) (end 174.4 104.4) (width 0.2) (layer "B.Cu") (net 18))
 (segment (start 163.66 106.46) (end 165.74 106.46) (width 0.2) (layer "B.Cu") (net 18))
 (segment (start 178.8 101.335255) (end 176.867628 103.267628) (width 0.2) (layer "B.Cu") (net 18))
 (segment (start 165.74 106.46) (end 167.8 104.4) (width 0.2) (layer "B.Cu") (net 18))
 (segment (start 179.6 93.2) (end 179.6 94.4) (width 0.2) (layer "F.Cu") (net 6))
 (via (at 179.6 93.2) (size 0.6) (drill 0.3) (layers "F.Cu" "B.Cu") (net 6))
 (segment (start 179.6 102.52) (end 179.6 93.2) (width 0.2) (layer "B.Cu") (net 6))
 (segment (start 175.66 106.46) (end 179.6 102.52) (width 0.2) (layer "B.Cu") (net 6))
 (segment (start 180.4 93.2) (end 180.4 94.4) (width 0.2) (layer "F.Cu") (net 8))
 (via (at 180.4 93.2) (size 0.6) (drill 0.3) (layers "F.Cu" "B.Cu") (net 8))
 (segment (start 187.66 106.46) (end 185.2 104) (width 0.2) (layer "B.Cu") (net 8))
 (segment (start 185.2 104) (end 183.6 104) (width 0.2) (layer "B.Cu") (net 8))
 (segment (start 180.4 100.8) (end 180.4 93.2) (width 0.2) (layer "B.Cu") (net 8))
 (segment (start 183.6 104) (end 180.4 100.8) (width 0.2) (layer "B.Cu") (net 8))
 (segment (start 181.2 93.2) (end 181.2 94.4) (width 0.2) (layer "F.Cu") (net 26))
 (via (at 181.2 93.2) (size 0.6) (drill 0.3) (layers "F.Cu" "B.Cu") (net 26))
 (segment (start 189.965 105.035) (end 187.73 102.8) (width 0.2) (layer "B.Cu") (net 26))
 (segment (start 183.6 102.8) (end 181.2 100.4) (width 0.2) (layer "B.Cu") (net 26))
 (segment (start 181.2 100.4) (end 181.2 93.2) (width 0.2) (layer "B.Cu") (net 26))
 (segment (start 198.235 105.035) (end 189.965 105.035) (width 0.2) (layer "B.Cu") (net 26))
 (segment (start 183.6 102.8) (end 187.73 102.8) (width 0.2) (layer "B.Cu") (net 26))
 (segment (start 199.66 106.46) (end 198.235 105.035) (width 0.2) (layer "B.Cu") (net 26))
 (segment (start 190.165 100.965) (end 189.4 100.2) (width 0.2) (layer "F.Cu") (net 19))
 (segment (start 192.507628 100.707628) (end 192.250256 100.965) (width 0.2) (layer "F.Cu") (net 19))
 (segment (start 185.05 100.2) (end 181.45 96.6) (width 0.2) (layer "F.Cu") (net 19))
 (segment (start 175.7 96.9) (end 175.5 96.9) (width 0.2) (layer "F.Cu") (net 19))
 (segment (start 194.2 97) (end 194.2 99.015255) (width 0.2) (layer "F.Cu") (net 19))
 (segment (start 189.4 100.2) (end 185.05 100.2) (width 0.2) (layer "F.Cu") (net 19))
 (segment (start 171.6 99.8) (end 170.8 99) (width 0.2) (layer "F.Cu") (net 19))
 (segment (start 194.2 99.015255) (end 192.507628 100.707628) (width 0.2) (layer "F.Cu") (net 19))
 (segment (start 170.8 99) (end 170.8 97.8) (width 0.2) (layer "F.Cu") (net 19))
 (segment (start 176 96.6) (end 175.7 96.9) (width 0.2) (layer "F.Cu") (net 19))
 (segment (start 192.250256 100.965) (end 190.165 100.965) (width 0.2) (layer "F.Cu") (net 19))
 (segment (start 172.6 99.8) (end 171.6 99.8) (width 0.2) (layer "F.Cu") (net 19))
 (segment (start 175.5 96.9) (end 172.6 99.8) (width 0.2) (layer "F.Cu") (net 19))
 (segment (start 181.45 96.6) (end 176 96.6) (width 0.2) (layer "F.Cu") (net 19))
 (segment (start 171.6 97.8) (end 171.6 98.6) (width 0.2) (layer "F.Cu") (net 21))
 (segment (start 171.6 98.6) (end 171.7 98.7) (width 0.2) (layer "F.Cu") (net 21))
 (segment (start 173.134314 98.7) (end 175.634314 96.2) (width 0.2) (layer "F.Cu") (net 21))
 (segment (start 195 95.675) (end 196.325 97) (width 0.2) (layer "F.Cu") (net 21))
 (segment (start 193.525 95.675) (end 195 95.675) (width 0.2) (layer "F.Cu") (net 21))
 (segment (start 196.325 97) (end 206.2 97) (width 0.2) (layer "F.Cu") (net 21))
 (segment (start 175.634314 96.2) (end 182.2 96.2) (width 0.2) (layer "F.Cu") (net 21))
 (segment (start 171.7 98.7) (end 173.134314 98.7) (width 0.2) (layer "F.Cu") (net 21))
 (segment (start 187.485 98.115) (end 191.085 98.115) (width 0.2) (layer "F.Cu") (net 21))
 (segment (start 184.585 98.585) (end 186.985 98.585) (width 0.2) (layer "F.Cu") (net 21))
 (segment (start 186.985 98.585) (end 187 98.6) (width 0.2) (layer "F.Cu") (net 21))
 (segment (start 182.2 96.2) (end 184.585 98.585) (width 0.2) (layer "F.Cu") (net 21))
 (segment (start 187 98.6) (end 187.485 98.115) (width 0.2) (layer "F.Cu") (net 21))
 (segment (start 191.085 98.115) (end 193.525 95.675) (width 0.2) (layer "F.Cu") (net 21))
 (segment (start 205.525 95.675) (end 207.875 95.675) (width 0.2) (layer "F.Cu") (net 1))
 (segment (start 188 96.2) (end 192.434314 96.2) (width 0.2) (layer "F.Cu") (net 1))
 (segment (start 186.926 95.126) (end 188 96.2) (width 0.2) (layer "F.Cu") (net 1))
 (segment (start 172.4 97.8) (end 174.9 95.3) (width 0.2) (layer "F.Cu") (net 1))
 (segment (start 183.7 95.3) (end 183.874 95.126) (width 0.2) (layer "F.Cu") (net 1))
 (segment (start 174.9 95.3) (end 183.7 95.3) (width 0.2) (layer "F.Cu") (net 1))
 (segment (start 195.2 95.275) (end 195.81 95.885) (width 0.2) (layer "F.Cu") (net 1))
 (segment (start 192.434314 96.2) (end 193.359314 95.275) (width 0.2) (layer "F.Cu") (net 1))
 (segment (start 207.875 95.675) (end 209.2 97) (width 0.2) (layer "F.Cu") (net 1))
 (segment (start 209.2 97) (end 218.2 97) (width 0.2) (layer "F.Cu") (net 1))
 (segment (start 195.81 95.885) (end 205.315 95.885) (width 0.2) (layer "F.Cu") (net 1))
 (segment (start 183.874 95.126) (end 186.926 95.126) (width 0.2) (layer "F.Cu") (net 1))
 (segment (start 193.359314 95.275) (end 195.2 95.275) (width 0.2) (layer "F.Cu") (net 1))
 (segment (start 205.315 95.885) (end 205.525 95.675) (width 0.2) (layer "F.Cu") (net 1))
 (segment (start 177.985785 91) (end 178.185785 90.8) (width 0.2) (layer "F.Cu") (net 20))
 (segment (start 179.414215 91.2) (end 191.2 91.2) (width 0.2) (layer "F.Cu") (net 20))
 (segment (start 170.8 93.6) (end 173.4 91) (width 0.2) (layer "F.Cu") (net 20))
 (segment (start 191.2 91.2) (end 191.66 91.66) (width 0.2) (layer "F.Cu") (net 20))
 (segment (start 170.8 94.4) (end 170.8 93.6) (width 0.2) (layer "F.Cu") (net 20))
 (segment (start 191.66 91.66) (end 191.66 94.46) (width 0.2) (layer "F.Cu") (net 20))
 (segment (start 178.185785 90.8) (end 179.014215 90.8) (width 0.2) (layer "F.Cu") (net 20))
 (segment (start 173.4 91) (end 177.985785 91) (width 0.2) (layer "F.Cu") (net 20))
 (segment (start 179.014215 90.8) (end 179.414215 91.2) (width 0.2) (layer "F.Cu") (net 20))
 (segment (start 190.8 92) (end 190.4 91.6) (width 0.2) (layer "F.Cu") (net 22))
 (segment (start 178.151471 91.4) (end 173.8 91.4) (width 0.2) (layer "F.Cu") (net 22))
 (segment (start 178.848529 91.2) (end 178.351471 91.2) (width 0.2) (layer "F.Cu") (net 22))
 (segment (start 173.8 91.4) (end 171.6 93.6) (width 0.2) (layer "F.Cu") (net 22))
 (segment (start 178.351471 91.2) (end 178.151471 91.4) (width 0.2) (layer "F.Cu") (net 22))
 (segment (start 179.2 91.551471) (end 178.848529 91.2) (width 0.2) (layer "F.Cu") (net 22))
 (segment (start 190.4 91.6) (end 179.2 91.6) (width 0.2) (layer "F.Cu") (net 22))
 (segment (start 171.6 93.6) (end 171.6 94.4) (width 0.2) (layer "F.Cu") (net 22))
 (segment (start 179.2 91.6) (end 179.2 91.551471) (width 0.2) (layer "F.Cu") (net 22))
 (via (at 190.8 92) (size 0.6) (drill 0.3) (layers "F.Cu" "B.Cu") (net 22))
 (segment (start 201.2 92) (end 203.66 94.46) (width 0.2) (layer "B.Cu") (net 22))
 (segment (start 190.8 92) (end 201.2 92) (width 0.2) (layer "B.Cu") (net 22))
 (segment (start 175.8 91.8) (end 178.6 91.8) (width 0.2) (layer "F.Cu") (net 2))
 (segment (start 172.4 94.4) (end 173.2 94.4) (width 0.2) (layer "F.Cu") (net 2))
 (segment (start 173.2 94.4) (end 175.8 91.8) (width 0.2) (layer "F.Cu") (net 2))
 (via (at 178.6 91.8) (size 0.6) (drill 0.3) (layers "F.Cu" "B.Cu") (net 2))
 (segment (start 190.2 91.4) (end 189.8 91.8) (width 0.2) (layer "B.Cu") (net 2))
 (segment (start 189.8 91.8) (end 178.6 91.8) (width 0.2) (layer "B.Cu") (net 2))
 (segment (start 215.66 94.46) (end 212.6 91.4) (width 0.2) (layer "B.Cu") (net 2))
 (segment (start 212.6 91.4) (end 190.2 91.4) (width 0.2) (layer "B.Cu") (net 2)))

